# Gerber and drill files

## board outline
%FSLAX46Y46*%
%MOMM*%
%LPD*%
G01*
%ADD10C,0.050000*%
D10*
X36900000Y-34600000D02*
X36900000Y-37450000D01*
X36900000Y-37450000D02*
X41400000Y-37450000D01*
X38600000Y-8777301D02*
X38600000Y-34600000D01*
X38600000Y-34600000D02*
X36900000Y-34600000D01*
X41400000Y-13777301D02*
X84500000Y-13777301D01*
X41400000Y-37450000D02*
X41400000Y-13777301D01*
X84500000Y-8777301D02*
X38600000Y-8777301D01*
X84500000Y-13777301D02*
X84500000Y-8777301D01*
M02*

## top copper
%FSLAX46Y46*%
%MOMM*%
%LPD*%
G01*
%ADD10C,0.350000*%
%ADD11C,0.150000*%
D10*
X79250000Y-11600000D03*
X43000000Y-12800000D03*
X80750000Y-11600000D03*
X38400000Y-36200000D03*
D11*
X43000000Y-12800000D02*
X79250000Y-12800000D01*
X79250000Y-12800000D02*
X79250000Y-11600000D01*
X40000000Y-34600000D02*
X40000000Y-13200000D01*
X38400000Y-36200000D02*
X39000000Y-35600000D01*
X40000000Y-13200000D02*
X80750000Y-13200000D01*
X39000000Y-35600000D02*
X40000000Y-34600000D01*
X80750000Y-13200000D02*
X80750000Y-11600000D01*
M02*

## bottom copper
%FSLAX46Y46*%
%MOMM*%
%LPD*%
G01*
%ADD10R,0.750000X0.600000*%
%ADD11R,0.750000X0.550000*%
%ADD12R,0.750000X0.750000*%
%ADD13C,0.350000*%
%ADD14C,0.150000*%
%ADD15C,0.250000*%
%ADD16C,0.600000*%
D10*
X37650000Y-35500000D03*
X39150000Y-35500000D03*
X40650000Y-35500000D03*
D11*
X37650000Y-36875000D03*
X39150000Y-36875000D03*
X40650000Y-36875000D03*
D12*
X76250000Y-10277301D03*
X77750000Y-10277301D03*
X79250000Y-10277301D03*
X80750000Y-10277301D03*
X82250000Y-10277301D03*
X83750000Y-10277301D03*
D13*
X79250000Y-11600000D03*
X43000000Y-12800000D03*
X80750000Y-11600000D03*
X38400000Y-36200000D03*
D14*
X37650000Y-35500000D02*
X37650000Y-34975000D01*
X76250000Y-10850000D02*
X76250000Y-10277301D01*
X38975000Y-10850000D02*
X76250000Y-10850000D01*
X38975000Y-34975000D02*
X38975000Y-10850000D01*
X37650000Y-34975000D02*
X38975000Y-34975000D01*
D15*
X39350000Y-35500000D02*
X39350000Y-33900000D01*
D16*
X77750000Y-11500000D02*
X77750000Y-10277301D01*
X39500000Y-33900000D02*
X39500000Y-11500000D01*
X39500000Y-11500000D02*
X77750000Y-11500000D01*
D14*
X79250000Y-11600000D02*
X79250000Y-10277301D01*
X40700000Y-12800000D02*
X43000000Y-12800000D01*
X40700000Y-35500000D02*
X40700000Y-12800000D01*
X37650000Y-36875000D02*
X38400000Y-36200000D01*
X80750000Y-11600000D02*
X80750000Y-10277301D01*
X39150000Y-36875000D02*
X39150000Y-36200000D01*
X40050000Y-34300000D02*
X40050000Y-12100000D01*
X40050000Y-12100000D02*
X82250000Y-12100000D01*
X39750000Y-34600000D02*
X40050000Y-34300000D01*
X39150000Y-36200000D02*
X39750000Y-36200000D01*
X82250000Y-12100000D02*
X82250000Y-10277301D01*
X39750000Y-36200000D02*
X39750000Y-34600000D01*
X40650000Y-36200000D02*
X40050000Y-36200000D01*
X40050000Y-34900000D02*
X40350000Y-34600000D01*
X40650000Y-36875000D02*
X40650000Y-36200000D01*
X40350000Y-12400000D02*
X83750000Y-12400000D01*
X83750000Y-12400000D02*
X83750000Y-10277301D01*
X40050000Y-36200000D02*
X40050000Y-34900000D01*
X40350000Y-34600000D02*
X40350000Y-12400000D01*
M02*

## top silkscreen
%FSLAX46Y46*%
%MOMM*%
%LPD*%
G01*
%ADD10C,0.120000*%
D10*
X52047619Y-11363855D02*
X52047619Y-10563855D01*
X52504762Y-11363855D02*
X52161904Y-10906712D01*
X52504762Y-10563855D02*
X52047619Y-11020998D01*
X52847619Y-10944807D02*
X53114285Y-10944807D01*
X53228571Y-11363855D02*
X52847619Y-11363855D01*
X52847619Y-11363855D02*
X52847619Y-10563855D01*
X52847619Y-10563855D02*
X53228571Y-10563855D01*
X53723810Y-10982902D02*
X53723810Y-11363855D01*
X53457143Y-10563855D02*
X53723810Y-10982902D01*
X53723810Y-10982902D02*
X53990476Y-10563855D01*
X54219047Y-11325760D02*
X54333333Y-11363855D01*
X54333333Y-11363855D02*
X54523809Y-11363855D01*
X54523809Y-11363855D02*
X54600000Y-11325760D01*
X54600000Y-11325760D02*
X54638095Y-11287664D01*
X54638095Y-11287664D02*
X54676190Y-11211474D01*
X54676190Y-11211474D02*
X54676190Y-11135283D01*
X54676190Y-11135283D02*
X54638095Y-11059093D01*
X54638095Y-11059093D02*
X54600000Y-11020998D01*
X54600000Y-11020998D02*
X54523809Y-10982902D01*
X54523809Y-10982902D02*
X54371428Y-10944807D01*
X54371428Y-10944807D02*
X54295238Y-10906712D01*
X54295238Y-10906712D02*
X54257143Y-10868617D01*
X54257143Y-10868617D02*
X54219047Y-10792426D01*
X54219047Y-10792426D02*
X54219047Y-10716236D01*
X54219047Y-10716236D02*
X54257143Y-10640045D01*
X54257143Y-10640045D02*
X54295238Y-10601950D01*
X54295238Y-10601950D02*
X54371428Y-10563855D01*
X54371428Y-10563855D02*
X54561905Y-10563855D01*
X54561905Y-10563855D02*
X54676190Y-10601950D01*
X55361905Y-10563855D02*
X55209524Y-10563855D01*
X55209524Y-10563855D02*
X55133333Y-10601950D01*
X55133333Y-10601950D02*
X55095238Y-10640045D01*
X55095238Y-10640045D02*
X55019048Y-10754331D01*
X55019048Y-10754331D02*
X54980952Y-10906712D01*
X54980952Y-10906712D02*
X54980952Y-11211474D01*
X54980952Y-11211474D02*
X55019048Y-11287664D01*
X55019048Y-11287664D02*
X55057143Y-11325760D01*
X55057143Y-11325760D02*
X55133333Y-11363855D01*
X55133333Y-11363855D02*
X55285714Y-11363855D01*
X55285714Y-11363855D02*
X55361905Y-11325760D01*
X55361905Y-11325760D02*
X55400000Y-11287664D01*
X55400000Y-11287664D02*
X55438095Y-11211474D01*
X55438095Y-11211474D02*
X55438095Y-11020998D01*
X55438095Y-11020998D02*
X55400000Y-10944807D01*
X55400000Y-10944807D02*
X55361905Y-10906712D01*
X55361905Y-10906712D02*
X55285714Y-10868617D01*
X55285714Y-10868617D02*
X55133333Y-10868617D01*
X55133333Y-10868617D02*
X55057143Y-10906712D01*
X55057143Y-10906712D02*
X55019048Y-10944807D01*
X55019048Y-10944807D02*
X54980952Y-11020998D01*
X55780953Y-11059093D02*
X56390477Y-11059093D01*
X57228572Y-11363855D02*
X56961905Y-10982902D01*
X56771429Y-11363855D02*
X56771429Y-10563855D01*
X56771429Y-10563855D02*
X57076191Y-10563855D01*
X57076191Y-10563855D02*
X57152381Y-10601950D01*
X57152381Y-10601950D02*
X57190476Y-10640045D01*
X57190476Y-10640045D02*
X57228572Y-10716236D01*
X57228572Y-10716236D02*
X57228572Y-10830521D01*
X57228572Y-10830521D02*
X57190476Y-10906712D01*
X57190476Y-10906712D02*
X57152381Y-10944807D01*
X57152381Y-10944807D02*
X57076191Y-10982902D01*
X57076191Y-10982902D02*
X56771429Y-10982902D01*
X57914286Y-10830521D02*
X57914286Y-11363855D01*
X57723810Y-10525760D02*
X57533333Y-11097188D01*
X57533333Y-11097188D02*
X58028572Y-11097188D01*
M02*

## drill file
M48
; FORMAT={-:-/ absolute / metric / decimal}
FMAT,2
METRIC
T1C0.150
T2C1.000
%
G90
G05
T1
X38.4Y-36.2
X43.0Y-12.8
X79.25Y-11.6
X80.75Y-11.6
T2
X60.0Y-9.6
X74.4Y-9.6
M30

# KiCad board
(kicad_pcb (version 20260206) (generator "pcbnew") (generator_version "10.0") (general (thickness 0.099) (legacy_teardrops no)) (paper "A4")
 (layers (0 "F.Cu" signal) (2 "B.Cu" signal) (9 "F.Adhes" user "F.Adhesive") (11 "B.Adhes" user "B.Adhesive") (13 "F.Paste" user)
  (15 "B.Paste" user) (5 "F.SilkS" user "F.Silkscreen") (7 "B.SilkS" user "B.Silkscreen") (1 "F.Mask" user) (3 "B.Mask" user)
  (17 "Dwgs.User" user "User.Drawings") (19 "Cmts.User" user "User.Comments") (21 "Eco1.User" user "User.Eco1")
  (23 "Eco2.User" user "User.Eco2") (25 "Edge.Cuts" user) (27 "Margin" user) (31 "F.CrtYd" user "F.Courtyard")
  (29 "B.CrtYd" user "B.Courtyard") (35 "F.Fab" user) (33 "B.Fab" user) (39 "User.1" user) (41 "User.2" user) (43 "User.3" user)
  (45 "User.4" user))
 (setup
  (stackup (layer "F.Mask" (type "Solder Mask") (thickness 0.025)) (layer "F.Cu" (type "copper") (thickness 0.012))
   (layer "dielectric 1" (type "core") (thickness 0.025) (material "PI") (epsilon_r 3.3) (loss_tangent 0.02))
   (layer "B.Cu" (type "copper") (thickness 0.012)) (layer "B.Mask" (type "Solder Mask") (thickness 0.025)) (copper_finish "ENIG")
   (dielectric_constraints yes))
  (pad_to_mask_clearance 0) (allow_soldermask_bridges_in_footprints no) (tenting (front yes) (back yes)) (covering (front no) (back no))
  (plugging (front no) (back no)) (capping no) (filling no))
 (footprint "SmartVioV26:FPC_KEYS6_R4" (layer "F.Cu") (at 0 0)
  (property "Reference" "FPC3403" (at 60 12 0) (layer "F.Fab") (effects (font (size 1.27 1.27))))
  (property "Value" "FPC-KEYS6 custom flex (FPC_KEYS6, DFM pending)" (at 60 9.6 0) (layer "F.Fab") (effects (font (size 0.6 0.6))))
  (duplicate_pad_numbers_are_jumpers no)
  (pad "" np_thru_hole circle (at 60 9.6) (size 1 1) (drill 1) (layers "*.Cu" "*.Mask"))
  (pad "" np_thru_hole circle (at 74.4 9.6) (size 1 1) (drill 1) (layers "*.Cu" "*.Mask"))
  (pad "S1" smd rect (at 37.65 35.5) (size 0.75 0.6) (layers "B.Cu" "B.Mask") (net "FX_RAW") (solder_mask_margin 0.1)
   (thermal_bridge_angle 45))
  (pad "S2" smd rect (at 39.15 35.5) (size 0.75 0.6) (layers "B.Cu" "B.Mask") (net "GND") (solder_mask_margin 0.1) (thermal_bridge_angle 45))
  (pad "S3" smd rect (at 40.65 35.5) (size 0.75 0.6) (layers "B.Cu" "B.Mask") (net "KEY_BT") (solder_mask_margin 0.1)
   (thermal_bridge_angle 45))
  (pad "S4" smd rect (at 37.65 36.875) (size 0.75 0.55) (layers "B.Cu" "B.Mask") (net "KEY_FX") (solder_mask_margin 0.1)
   (thermal_bridge_angle 45))
  (pad "S5" smd rect (at 39.15 36.875) (size 0.75 0.55) (layers "B.Cu" "B.Mask") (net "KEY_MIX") (solder_mask_margin 0.1)
   (thermal_bridge_angle 45))
  (pad "S6" smd rect (at 40.65 36.875) (size 0.75 0.55) (layers "B.Cu" "B.Mask") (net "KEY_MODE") (solder_mask_margin 0.1)
   (thermal_bridge_angle 45))
  (pad "T1" smd rect (at 76.25 10.277301) (size 0.75 0.75) (layers "B.Cu" "B.Mask") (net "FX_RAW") (solder_mask_margin 0.1)
   (thermal_bridge_angle 45))
  (pad "T2" smd rect (at 77.75 10.277301) (size 0.75 0.75) (layers "B.Cu" "B.Mask") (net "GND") (solder_mask_margin 0.1)
   (thermal_bridge_angle 45))
  (pad "T3" smd rect (at 79.25 10.277301) (size 0.75 0.75) (layers "B.Cu" "B.Mask") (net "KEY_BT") (solder_mask_margin 0.1)
   (thermal_bridge_angle 45))
  (pad "T4" smd rect (at 80.75 10.277301) (size 0.75 0.75) (layers "B.Cu" "B.Mask") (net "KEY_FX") (solder_mask_margin 0.1)
   (thermal_bridge_angle 45))
  (pad "T5" smd rect (at 82.25 10.277301) (size 0.75 0.75) (layers "B.Cu" "B.Mask") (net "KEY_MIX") (solder_mask_margin 0.1)
   (thermal_bridge_angle 45))
  (pad "T6" smd rect (at 83.75 10.277301) (size 0.75 0.75) (layers "B.Cu" "B.Mask") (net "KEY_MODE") (solder_mask_margin 0.1)
   (thermal_bridge_angle 45)))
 (gr_line (start 36.9 34.6) (end 36.9 37.45) (stroke (width 0.05) (type default)) (layer "Edge.Cuts"))
 (gr_line (start 36.9 37.45) (end 41.4 37.45) (stroke (width 0.05) (type default)) (layer "Edge.Cuts"))
 (gr_line (start 38.6 8.777301) (end 38.6 34.6) (stroke (width 0.05) (type default)) (layer "Edge.Cuts"))
 (gr_line (start 38.6 34.6) (end 36.9 34.6) (stroke (width 0.05) (type default)) (layer "Edge.Cuts"))
 (gr_line (start 41.4 13.777301) (end 84.5 13.777301) (stroke (width 0.05) (type default)) (layer "Edge.Cuts"))
 (gr_line (start 41.4 37.45) (end 41.4 13.777301) (stroke (width 0.05) (type default)) (layer "Edge.Cuts"))
 (gr_line (start 84.5 8.777301) (end 38.6 8.777301) (stroke (width 0.05) (type default)) (layer "Edge.Cuts"))
 (gr_line (start 84.5 13.777301) (end 84.5 8.777301) (stroke (width 0.05) (type default)) (layer "Edge.Cuts"))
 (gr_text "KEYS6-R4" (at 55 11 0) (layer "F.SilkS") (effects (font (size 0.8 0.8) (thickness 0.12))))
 (segment (start 37.65 35.5) (end 37.65 34.975) (width 0.15) (layer "B.Cu") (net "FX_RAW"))
 (segment (start 76.25 10.85) (end 76.25 10.277301) (width 0.15) (layer "B.Cu") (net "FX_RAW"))
 (segment (start 38.975 10.85) (end 76.25 10.85) (width 0.15) (layer "B.Cu") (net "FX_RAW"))
 (segment (start 38.975 34.975) (end 38.975 10.85) (width 0.15) (layer "B.Cu") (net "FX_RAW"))
 (segment (start 37.65 34.975) (end 38.975 34.975) (width 0.15) (layer "B.Cu") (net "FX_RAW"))
 (segment (start 39.35 35.5) (end 39.35 33.9) (width 0.25) (layer "B.Cu") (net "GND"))
 (segment (start 77.75 11.5) (end 77.75 10.277301) (width 0.6) (layer "B.Cu") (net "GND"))
 (segment (start 39.5 33.9) (end 39.5 11.5) (width 0.6) (layer "B.Cu") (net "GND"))
 (segment (start 39.5 11.5) (end 77.75 11.5) (width 0.6) (layer "B.Cu") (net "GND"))
 (segment (start 43 12.8) (end 79.25 12.8) (width 0.15) (layer "F.Cu") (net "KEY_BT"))
 (segment (start 79.25 12.8) (end 79.25 11.6) (width 0.15) (layer "F.Cu") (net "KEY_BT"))
 (via (at 79.25 11.6) (size 0.35) (drill 0.15) (layers "F.Cu" "B.Cu") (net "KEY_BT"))
 (via (at 43 12.8) (size 0.35) (drill 0.15) (layers "F.Cu" "B.Cu") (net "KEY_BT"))
 (segment (start 79.25 11.6) (end 79.25 10.277301) (width 0.15) (layer "B.Cu") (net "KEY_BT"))
 (segment (start 40.7 12.8) (end 43 12.8) (width 0.15) (layer "B.Cu") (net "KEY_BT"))
 (segment (start 40.7 35.5) (end 40.7 12.8) (width 0.15) (layer "B.Cu") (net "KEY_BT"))
 (segment (start 40 34.6) (end 40 13.2) (width 0.15) (layer "F.Cu") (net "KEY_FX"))
 (segment (start 38.4 36.2) (end 39 35.6) (width 0.15) (layer "F.Cu") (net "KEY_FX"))
 (segment (start 40 13.2) (end 80.75 13.2) (width 0.15) (layer "F.Cu") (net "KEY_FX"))
 (segment (start 39 35.6) (end 40 34.6) (width 0.15) (layer "F.Cu") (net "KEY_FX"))
 (segment (start 80.75 13.2) (end 80.75 11.6) (width 0.15) (layer "F.Cu") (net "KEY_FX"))
 (via (at 80.75 11.6) (size 0.35) (drill 0.15) (layers "F.Cu" "B.Cu") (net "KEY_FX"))
 (via (at 38.4 36.2) (size 0.35) (drill 0.15) (layers "F.Cu" "B.Cu") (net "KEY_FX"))
 (segment (start 37.65 36.875) (end 38.4 36.2) (width 0.15) (layer "B.Cu") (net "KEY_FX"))
 (segment (start 80.75 11.6) (end 80.75 10.277301) (width 0.15) (layer "B.Cu") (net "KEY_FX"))
 (segment (start 39.15 36.875) (end 39.15 36.2) (width 0.15) (layer "B.Cu") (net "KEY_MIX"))
 (segment (start 40.05 34.3) (end 40.05 12.1) (width 0.15) (layer "B.Cu") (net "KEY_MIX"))
 (segment (start 40.05 12.1) (end 82.25 12.1) (width 0.15) (layer "B.Cu") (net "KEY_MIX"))
 (segment (start 39.75 34.6) (end 40.05 34.3) (width 0.15) (layer "B.Cu") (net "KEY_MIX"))
 (segment (start 39.15 36.2) (end 39.75 36.2) (width 0.15) (layer "B.Cu") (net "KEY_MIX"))
 (segment (start 82.25 12.1) (end 82.25 10.277301) (width 0.15) (layer "B.Cu") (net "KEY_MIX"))
 (segment (start 39.75 36.2) (end 39.75 34.6) (width 0.15) (layer "B.Cu") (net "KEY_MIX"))
 (segment (start 40.65 36.2) (end 40.05 36.2) (width 0.15) (layer "B.Cu") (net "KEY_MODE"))
 (segment (start 40.05 34.9) (end 40.35 34.6) (width 0.15) (layer "B.Cu") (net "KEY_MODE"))
 (segment (start 40.65 36.875) (end 40.65 36.2) (width 0.15) (layer "B.Cu") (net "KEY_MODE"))
 (segment (start 40.35 12.4) (end 83.75 12.4) (width 0.15) (layer "B.Cu") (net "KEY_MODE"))
 (segment (start 83.75 12.4) (end 83.75 10.277301) (width 0.15) (layer "B.Cu") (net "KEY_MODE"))
 (segment (start 40.05 36.2) (end 40.05 34.9) (width 0.15) (layer "B.Cu") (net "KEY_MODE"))
 (segment (start 40.35 34.6) (end 40.35 12.4) (width 0.15) (layer "B.Cu") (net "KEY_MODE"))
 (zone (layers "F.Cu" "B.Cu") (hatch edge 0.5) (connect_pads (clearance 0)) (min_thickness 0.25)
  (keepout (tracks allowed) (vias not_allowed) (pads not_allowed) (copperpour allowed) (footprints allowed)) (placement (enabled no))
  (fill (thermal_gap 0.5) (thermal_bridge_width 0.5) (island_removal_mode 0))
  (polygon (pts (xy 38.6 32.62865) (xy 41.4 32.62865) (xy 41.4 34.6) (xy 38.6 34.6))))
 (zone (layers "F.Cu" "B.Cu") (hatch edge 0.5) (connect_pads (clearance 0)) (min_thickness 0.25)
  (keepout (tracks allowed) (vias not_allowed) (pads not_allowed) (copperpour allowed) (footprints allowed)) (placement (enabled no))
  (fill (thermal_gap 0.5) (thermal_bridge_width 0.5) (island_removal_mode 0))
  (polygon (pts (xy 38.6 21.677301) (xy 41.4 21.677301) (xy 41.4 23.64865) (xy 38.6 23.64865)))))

